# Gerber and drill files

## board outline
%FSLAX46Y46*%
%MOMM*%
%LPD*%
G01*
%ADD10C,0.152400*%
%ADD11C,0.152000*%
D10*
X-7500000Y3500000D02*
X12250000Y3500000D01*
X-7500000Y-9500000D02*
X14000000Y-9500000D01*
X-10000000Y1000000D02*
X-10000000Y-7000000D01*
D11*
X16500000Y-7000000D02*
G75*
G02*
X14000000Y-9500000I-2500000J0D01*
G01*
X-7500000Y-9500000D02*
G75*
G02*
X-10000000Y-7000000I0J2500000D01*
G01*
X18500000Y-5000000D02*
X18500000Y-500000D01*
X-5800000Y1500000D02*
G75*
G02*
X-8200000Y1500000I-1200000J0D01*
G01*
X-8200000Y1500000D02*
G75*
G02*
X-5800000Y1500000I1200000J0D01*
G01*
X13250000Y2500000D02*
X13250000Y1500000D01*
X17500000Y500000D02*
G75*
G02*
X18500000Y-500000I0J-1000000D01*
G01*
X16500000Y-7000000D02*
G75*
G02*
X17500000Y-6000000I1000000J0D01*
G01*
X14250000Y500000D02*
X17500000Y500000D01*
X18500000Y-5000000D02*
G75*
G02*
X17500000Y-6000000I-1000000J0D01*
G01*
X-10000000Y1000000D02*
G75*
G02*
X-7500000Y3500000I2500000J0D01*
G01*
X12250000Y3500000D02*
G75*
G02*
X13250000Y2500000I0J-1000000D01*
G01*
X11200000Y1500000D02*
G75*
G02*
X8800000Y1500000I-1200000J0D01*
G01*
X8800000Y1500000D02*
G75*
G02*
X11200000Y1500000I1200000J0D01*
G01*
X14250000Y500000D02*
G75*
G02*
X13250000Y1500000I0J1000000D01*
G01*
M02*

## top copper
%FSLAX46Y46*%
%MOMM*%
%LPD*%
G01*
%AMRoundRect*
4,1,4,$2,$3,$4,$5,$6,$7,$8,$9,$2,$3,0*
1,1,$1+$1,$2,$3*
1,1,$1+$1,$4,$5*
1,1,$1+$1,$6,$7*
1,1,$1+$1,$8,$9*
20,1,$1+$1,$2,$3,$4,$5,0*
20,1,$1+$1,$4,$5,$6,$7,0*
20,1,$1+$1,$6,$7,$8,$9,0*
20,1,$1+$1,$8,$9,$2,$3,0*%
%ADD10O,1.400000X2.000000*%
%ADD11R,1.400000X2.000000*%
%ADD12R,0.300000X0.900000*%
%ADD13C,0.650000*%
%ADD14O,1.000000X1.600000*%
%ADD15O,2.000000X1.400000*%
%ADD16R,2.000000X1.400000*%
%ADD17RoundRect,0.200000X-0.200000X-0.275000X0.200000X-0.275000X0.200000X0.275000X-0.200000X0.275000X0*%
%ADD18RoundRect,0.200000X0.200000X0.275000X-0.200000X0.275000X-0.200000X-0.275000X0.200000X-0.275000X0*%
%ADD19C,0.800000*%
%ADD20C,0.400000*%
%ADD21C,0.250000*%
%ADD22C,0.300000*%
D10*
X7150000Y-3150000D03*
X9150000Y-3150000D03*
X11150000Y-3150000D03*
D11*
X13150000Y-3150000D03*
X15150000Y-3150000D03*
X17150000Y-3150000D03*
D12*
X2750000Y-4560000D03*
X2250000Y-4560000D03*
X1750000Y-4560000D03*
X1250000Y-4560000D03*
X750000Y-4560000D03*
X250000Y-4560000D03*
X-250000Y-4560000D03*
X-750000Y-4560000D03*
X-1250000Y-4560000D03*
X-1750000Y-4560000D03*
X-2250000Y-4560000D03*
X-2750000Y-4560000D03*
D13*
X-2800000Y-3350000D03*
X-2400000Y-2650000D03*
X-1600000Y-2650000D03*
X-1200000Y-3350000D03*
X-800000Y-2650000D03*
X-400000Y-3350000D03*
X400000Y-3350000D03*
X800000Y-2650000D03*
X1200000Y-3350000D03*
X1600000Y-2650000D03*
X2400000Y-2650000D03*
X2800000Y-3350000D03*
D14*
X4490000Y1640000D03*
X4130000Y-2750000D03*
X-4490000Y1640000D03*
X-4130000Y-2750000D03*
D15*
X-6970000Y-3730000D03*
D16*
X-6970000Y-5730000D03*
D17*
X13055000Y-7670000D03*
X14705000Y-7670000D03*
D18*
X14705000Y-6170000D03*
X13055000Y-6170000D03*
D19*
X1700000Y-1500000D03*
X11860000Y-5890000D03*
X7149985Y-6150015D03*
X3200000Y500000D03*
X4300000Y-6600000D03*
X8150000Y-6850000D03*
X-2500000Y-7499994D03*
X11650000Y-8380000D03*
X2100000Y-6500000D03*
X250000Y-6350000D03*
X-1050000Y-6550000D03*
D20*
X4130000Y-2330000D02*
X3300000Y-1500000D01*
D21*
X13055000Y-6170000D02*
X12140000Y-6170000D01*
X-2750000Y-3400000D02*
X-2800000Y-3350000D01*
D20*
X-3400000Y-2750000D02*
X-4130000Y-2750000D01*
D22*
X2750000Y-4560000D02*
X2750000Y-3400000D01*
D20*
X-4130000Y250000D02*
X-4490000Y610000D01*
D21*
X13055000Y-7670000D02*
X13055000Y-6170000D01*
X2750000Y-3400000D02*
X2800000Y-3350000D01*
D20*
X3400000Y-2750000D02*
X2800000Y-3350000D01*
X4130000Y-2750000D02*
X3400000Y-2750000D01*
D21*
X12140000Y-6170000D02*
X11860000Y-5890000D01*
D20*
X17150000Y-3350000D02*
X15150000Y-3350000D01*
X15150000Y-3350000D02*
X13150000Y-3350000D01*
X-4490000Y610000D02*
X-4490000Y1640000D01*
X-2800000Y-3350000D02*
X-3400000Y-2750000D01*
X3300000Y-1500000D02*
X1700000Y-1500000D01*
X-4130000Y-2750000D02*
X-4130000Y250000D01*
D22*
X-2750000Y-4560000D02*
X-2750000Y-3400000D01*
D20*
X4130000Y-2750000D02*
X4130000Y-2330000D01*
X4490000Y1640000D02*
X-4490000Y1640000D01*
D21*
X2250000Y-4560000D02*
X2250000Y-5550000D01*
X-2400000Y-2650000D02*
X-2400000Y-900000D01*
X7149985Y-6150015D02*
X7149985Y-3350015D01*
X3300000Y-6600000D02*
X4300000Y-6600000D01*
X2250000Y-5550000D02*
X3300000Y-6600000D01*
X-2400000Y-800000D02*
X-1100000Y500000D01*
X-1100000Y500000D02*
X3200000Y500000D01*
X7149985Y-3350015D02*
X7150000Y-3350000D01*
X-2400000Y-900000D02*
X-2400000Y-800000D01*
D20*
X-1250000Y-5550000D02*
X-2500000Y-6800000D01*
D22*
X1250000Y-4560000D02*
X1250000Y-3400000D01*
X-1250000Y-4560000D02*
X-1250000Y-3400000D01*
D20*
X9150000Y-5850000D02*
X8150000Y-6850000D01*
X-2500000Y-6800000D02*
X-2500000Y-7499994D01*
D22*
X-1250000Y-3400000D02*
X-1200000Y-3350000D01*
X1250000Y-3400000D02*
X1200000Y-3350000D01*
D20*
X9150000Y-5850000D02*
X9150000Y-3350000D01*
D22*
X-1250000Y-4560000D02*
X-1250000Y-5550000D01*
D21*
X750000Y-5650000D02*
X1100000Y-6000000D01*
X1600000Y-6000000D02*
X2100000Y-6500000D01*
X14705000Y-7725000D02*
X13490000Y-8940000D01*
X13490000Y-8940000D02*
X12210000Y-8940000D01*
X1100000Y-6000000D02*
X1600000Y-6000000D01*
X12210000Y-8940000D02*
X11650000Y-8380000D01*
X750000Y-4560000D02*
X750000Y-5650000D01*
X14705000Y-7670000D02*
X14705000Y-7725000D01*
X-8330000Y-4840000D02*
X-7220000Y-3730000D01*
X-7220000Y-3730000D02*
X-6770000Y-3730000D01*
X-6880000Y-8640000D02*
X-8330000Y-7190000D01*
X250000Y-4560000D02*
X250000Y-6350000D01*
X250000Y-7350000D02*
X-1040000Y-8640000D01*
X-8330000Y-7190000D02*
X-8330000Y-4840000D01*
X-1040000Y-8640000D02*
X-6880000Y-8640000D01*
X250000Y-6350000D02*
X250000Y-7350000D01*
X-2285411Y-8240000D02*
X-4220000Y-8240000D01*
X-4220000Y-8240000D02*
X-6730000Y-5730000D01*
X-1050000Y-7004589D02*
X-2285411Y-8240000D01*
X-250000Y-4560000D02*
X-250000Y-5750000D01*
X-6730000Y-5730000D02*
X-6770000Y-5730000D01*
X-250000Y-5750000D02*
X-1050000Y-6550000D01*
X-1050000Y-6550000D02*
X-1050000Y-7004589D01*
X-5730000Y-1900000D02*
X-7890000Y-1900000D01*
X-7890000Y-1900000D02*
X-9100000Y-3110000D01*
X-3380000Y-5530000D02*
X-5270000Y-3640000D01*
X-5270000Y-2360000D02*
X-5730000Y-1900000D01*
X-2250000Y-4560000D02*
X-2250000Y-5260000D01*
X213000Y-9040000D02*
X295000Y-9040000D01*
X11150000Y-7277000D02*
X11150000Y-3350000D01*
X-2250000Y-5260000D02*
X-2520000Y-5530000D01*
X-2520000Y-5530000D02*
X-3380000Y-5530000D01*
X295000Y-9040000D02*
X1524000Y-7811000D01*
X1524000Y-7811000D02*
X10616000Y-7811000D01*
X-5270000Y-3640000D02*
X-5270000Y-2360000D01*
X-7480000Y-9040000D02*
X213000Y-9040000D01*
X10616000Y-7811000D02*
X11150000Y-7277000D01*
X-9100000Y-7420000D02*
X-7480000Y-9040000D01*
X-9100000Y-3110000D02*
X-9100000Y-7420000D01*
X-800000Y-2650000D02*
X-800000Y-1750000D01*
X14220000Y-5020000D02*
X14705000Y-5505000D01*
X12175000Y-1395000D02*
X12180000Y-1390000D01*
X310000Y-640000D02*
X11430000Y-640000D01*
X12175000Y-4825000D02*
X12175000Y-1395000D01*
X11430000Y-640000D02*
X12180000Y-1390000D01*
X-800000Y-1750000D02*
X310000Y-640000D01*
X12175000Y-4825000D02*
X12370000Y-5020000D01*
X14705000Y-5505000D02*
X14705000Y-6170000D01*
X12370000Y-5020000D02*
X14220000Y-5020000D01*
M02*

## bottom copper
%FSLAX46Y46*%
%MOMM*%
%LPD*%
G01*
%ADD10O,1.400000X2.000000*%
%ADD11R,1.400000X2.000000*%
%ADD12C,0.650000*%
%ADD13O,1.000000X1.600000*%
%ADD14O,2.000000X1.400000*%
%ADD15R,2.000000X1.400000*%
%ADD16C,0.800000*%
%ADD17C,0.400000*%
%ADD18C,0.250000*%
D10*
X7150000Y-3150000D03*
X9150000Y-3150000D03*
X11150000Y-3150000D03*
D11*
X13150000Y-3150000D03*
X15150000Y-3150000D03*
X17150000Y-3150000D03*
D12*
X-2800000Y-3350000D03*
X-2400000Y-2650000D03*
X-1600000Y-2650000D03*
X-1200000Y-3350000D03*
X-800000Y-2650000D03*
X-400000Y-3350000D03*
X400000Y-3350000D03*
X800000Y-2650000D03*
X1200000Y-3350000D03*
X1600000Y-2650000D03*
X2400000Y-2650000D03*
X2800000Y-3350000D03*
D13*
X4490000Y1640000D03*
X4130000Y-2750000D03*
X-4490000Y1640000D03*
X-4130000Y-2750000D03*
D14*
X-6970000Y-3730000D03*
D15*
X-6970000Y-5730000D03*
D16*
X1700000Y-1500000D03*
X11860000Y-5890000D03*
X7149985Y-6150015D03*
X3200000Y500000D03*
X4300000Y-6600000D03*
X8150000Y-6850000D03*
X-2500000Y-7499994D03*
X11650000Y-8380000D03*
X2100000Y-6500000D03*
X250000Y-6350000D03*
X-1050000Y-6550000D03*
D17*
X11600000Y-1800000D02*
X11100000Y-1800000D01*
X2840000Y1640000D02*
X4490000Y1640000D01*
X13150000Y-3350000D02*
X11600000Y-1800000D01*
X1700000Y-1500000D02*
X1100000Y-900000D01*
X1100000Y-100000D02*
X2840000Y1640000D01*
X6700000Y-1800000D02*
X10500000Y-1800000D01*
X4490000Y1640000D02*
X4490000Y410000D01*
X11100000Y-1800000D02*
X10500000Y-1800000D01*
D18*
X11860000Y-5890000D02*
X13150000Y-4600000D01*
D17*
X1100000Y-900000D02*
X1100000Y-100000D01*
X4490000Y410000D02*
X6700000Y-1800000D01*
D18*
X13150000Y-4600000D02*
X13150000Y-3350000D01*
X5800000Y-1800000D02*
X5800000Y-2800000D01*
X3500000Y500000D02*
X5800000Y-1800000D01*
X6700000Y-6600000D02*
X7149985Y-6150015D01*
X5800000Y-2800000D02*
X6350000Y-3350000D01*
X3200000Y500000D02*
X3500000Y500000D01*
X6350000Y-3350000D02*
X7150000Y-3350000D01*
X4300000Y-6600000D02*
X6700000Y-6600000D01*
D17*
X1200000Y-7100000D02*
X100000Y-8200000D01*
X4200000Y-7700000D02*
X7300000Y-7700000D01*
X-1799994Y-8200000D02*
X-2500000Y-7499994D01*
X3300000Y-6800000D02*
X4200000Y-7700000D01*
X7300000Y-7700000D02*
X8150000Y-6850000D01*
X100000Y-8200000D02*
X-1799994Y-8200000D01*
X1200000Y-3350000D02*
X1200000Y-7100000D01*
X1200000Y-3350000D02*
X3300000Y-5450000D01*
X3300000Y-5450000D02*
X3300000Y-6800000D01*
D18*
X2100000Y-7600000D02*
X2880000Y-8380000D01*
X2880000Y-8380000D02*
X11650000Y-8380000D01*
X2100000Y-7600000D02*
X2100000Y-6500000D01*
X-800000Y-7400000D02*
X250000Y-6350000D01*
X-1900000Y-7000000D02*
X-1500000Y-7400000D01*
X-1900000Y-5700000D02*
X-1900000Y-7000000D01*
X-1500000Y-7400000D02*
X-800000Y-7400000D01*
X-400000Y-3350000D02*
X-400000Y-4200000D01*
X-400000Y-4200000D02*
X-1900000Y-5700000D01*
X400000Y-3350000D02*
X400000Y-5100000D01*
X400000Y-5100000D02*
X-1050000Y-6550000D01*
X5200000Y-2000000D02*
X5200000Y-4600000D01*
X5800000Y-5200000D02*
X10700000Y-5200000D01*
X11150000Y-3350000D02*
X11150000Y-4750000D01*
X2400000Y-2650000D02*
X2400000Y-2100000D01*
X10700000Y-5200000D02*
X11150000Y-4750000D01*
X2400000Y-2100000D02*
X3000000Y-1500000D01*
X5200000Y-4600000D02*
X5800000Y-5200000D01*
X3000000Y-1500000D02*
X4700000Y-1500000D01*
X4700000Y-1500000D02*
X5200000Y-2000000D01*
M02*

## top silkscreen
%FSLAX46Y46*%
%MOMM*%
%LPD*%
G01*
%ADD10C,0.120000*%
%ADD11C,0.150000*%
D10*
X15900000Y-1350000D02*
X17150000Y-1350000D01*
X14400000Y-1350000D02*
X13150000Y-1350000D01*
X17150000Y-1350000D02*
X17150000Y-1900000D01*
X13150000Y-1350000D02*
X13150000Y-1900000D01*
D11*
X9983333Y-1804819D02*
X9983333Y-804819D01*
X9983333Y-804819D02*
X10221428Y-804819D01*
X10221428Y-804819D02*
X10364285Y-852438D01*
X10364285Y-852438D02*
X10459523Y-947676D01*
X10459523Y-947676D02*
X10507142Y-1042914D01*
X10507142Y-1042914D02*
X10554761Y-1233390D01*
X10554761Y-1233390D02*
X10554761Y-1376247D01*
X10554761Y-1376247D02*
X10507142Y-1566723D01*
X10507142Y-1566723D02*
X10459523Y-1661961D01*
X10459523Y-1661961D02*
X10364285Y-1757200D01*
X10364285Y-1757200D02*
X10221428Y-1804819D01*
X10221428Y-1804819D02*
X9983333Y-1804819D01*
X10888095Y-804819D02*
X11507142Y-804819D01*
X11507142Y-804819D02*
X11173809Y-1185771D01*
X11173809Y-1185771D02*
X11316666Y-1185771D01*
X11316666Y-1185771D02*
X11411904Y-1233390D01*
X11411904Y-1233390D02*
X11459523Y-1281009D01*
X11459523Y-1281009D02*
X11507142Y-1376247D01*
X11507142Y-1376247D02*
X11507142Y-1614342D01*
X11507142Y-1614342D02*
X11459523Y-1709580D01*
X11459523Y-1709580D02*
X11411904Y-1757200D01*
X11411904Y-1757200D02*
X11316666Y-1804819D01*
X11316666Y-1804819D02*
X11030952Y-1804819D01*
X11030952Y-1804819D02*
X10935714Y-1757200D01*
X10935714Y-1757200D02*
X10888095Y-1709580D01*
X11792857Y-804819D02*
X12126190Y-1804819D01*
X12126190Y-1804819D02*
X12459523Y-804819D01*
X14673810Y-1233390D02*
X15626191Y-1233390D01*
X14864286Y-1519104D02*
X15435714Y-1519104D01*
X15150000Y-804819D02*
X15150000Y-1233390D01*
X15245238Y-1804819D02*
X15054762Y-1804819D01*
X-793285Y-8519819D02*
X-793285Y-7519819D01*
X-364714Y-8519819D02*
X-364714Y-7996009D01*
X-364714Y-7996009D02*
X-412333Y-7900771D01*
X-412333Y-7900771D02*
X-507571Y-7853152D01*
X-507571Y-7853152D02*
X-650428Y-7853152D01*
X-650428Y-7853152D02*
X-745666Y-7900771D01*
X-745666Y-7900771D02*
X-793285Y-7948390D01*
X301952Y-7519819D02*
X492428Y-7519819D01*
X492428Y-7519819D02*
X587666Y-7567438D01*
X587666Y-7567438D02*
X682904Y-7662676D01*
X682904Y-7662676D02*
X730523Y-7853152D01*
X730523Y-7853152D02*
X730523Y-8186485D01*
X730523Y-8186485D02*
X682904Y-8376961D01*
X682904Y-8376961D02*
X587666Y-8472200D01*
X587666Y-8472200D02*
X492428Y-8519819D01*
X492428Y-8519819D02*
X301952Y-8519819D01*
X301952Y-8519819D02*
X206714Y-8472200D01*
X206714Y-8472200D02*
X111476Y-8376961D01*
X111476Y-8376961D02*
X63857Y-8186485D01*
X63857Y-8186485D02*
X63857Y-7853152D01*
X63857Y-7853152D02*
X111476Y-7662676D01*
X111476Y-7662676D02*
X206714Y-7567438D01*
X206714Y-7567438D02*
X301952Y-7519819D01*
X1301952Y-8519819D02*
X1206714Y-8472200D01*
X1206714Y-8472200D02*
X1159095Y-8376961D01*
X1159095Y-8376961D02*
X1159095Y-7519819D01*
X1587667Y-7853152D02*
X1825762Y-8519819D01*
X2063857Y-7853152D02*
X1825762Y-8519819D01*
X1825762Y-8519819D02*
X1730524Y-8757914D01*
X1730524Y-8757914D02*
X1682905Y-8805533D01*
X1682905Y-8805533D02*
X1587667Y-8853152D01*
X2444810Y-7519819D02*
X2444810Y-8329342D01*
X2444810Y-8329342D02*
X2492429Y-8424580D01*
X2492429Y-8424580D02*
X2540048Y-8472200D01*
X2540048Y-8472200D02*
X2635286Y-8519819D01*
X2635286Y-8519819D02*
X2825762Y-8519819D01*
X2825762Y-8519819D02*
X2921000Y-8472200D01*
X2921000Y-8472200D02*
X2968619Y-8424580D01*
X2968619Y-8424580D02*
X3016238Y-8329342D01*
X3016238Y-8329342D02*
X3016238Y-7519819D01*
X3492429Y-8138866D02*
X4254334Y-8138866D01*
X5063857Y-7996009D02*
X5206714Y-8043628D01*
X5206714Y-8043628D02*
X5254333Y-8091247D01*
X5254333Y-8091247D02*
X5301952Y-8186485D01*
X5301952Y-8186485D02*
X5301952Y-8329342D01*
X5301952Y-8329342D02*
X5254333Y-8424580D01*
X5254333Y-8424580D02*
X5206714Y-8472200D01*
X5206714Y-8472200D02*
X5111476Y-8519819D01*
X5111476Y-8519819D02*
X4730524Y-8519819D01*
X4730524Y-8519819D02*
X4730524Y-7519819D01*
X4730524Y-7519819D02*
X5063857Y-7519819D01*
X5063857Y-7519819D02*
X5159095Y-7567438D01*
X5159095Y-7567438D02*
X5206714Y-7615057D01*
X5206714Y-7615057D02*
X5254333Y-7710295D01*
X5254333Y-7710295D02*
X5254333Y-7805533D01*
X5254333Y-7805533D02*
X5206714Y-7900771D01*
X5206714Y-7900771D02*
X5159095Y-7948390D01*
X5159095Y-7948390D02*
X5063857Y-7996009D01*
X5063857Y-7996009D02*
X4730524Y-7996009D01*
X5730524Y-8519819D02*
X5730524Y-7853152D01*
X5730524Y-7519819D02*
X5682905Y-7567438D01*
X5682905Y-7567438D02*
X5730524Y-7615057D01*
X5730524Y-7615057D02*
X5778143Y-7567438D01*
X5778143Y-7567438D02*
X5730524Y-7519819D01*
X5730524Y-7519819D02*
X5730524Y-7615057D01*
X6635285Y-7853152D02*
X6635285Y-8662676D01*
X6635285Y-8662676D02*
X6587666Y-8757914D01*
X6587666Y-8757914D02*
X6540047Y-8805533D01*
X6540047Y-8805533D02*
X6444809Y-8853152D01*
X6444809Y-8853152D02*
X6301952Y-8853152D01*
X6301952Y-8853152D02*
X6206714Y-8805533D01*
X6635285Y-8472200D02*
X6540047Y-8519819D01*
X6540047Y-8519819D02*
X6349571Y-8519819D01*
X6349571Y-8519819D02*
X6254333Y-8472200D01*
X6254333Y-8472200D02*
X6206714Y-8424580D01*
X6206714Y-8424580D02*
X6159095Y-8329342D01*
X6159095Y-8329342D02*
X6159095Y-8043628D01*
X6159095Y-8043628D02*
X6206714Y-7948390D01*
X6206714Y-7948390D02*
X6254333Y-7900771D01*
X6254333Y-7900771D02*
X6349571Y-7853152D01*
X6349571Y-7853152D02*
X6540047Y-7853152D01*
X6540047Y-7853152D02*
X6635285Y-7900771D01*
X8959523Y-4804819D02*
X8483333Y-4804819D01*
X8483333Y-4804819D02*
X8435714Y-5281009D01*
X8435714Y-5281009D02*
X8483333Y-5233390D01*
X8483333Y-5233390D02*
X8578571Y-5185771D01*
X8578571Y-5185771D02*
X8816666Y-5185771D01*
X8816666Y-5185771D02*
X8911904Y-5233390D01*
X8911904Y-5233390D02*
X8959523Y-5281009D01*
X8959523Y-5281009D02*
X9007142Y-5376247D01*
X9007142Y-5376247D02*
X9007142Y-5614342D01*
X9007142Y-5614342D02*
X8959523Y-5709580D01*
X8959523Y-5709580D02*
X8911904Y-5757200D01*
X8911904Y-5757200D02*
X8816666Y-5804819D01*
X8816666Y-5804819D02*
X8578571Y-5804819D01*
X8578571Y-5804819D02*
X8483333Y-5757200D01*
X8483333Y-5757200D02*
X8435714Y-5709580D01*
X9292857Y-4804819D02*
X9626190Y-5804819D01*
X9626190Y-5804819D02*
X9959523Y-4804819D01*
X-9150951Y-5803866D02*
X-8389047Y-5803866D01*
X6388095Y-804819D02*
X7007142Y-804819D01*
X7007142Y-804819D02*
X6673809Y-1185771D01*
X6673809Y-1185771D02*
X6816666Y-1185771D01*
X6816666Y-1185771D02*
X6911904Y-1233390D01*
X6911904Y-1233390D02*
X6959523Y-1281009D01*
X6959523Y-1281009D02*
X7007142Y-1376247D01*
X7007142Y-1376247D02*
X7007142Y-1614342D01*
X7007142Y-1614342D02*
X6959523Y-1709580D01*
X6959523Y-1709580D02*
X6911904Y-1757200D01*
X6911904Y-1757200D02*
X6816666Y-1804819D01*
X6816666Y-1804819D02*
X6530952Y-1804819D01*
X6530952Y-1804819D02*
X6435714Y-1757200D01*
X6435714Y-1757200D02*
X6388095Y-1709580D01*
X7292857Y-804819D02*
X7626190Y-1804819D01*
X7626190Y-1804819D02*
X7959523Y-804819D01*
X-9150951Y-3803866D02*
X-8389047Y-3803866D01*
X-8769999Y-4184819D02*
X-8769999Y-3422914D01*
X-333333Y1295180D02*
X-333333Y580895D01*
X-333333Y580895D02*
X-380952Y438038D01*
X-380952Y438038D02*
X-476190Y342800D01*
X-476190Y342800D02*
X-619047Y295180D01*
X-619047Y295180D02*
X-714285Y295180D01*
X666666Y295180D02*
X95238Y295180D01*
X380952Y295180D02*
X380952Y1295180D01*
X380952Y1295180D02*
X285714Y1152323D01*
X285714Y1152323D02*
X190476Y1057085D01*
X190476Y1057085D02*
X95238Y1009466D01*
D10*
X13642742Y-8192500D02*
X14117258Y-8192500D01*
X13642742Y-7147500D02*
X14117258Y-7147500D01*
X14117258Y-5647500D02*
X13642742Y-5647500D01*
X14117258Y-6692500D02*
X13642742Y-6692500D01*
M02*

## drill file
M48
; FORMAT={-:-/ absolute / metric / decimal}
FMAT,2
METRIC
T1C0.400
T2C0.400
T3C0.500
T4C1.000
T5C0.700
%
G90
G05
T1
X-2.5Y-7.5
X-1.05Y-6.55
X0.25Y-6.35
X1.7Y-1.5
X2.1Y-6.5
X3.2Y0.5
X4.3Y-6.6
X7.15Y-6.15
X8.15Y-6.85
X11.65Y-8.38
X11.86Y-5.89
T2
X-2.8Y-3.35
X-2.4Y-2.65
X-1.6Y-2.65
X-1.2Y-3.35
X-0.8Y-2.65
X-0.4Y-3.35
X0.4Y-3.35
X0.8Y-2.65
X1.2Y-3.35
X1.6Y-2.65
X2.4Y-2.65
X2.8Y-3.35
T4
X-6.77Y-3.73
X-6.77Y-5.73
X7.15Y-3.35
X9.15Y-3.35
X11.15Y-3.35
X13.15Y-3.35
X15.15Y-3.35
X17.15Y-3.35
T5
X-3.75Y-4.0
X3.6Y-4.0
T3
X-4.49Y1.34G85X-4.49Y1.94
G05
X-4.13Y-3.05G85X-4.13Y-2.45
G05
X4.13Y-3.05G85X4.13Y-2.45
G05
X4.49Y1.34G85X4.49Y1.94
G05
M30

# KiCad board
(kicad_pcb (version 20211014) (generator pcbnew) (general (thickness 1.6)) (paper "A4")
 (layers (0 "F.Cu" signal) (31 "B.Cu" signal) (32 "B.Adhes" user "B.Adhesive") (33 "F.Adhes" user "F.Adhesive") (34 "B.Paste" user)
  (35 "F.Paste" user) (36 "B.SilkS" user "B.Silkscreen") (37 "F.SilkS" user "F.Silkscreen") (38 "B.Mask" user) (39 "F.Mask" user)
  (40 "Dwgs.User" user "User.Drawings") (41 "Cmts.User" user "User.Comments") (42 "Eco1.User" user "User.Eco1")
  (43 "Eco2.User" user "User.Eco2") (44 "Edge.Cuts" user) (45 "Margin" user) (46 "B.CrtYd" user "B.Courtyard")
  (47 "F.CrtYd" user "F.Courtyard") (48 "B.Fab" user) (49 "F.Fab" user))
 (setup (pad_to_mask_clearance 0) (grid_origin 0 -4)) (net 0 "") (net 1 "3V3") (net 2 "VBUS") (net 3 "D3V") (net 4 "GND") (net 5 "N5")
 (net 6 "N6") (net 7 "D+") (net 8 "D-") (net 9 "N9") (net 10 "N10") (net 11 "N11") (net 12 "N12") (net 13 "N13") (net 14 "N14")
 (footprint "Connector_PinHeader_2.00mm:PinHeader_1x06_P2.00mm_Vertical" (layer "F.Cu") (at 7.15 3.35 90)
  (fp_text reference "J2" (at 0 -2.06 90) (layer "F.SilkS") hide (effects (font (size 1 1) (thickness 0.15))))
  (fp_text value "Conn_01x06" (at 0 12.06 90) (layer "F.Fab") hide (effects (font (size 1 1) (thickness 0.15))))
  (pad "1" thru_hole oval locked (at 0 0 90) (size 2 1.4) (drill 1 (offset 0.2 0)) (layers *.Cu *.Mask) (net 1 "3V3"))
  (pad "2" thru_hole oval locked (at 0 2 90) (size 2 1.4) (drill 1 (offset 0.2 0)) (layers *.Cu *.Mask) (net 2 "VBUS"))
  (pad "3" thru_hole oval locked (at 0 4 90) (size 2 1.4) (drill 1 (offset 0.2 0)) (layers *.Cu *.Mask) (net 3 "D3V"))
  (pad "4" thru_hole rect locked (at 0 6 90) (size 2 1.4) (drill 1 (offset 0.2 0)) (layers *.Cu *.Mask) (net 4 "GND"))
  (pad "5" thru_hole rect locked (at 0 8 90) (size 2 1.4) (drill 1 (offset 0.2 0)) (layers *.Cu *.Mask) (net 4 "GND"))
  (pad "6" thru_hole rect locked (at 0 10 90) (size 2 1.4) (drill 1 (offset 0.2 0)) (layers *.Cu *.Mask) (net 4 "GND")))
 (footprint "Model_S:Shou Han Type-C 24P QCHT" (layer "F.Cu") (at 0 -3.5 180)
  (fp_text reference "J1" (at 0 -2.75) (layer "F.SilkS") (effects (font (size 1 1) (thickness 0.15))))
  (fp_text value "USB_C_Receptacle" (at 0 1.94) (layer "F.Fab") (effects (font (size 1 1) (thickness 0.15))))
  (pad "" np_thru_hole circle locked (at -3.6 -7.5 180) (size 0.7 0.7) (drill 0.7) (layers *.Cu *.Mask))
  (pad "" np_thru_hole circle locked (at 3.75 -7.5 180) (size 0.7 0.7) (drill 0.7) (layers *.Cu *.Mask))
  (pad "A1" smd rect locked (at -2.75 -8.06 180) (size 0.3 0.9) (layers "F.Cu" "F.Paste" "F.Mask") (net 4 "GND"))
  (pad "A2" smd rect locked (at -2.25 -8.06 180) (size 0.3 0.9) (layers "F.Cu" "F.Paste" "F.Mask") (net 1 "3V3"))
  (pad "A3" smd rect locked (at -1.75 -8.06 180) (size 0.3 0.9) (layers "F.Cu" "F.Paste" "F.Mask") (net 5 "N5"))
  (pad "A4" smd rect locked (at -1.25 -8.06 180) (size 0.3 0.9) (layers "F.Cu" "F.Paste" "F.Mask") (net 2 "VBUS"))
  (pad "A5" smd rect locked (at -0.75 -8.06 180) (size 0.3 0.9) (layers "F.Cu" "F.Paste" "F.Mask") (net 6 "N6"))
  (pad "A6" smd rect locked (at -0.25 -8.06 180) (size 0.3 0.9) (layers "F.Cu" "F.Paste" "F.Mask") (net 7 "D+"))
  (pad "A7" smd rect locked (at 0.25 -8.06 180) (size 0.3 0.9) (layers "F.Cu" "F.Paste" "F.Mask") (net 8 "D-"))
  (pad "A8" smd rect locked (at 0.75 -8.06 180) (size 0.3 0.9) (layers "F.Cu" "F.Paste" "F.Mask") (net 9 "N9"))
  (pad "A9" smd rect locked (at 1.25 -8.06 180) (size 0.3 0.9) (layers "F.Cu" "F.Paste" "F.Mask") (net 2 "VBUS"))
  (pad "A10" smd rect locked (at 1.75 -8.06 180) (size 0.3 0.9) (layers "F.Cu" "F.Paste" "F.Mask") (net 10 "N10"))
  (pad "A11" smd rect locked (at 2.25 -8.06 180) (size 0.3 0.9) (layers "F.Cu" "F.Paste" "F.Mask") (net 3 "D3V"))
  (pad "A12" smd rect locked (at 2.75 -8.06 180) (size 0.3 0.9) (layers "F.Cu" "F.Paste" "F.Mask") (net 4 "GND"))
  (pad "B1" thru_hole circle locked (at 2.8 -6.85 180) (size 0.65 0.65) (drill 0.4) (layers *.Cu *.Mask) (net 4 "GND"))
  (pad "B2" thru_hole circle locked (at 2.4 -6.15 180) (size 0.65 0.65) (drill 0.4) (layers *.Cu *.Mask) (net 1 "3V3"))
  (pad "B3" thru_hole circle locked (at 1.6 -6.15 180) (size 0.65 0.65) (drill 0.4) (layers *.Cu *.Mask) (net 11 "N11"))
  (pad "B4" thru_hole circle locked (at 1.2 -6.85 180) (size 0.65 0.65) (drill 0.4) (layers *.Cu *.Mask) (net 2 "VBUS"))
  (pad "B5" thru_hole circle locked (at 0.8 -6.15 180) (size 0.65 0.65) (drill 0.4) (layers *.Cu *.Mask) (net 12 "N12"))
  (pad "B6" thru_hole circle locked (at 0.4 -6.85 180) (size 0.65 0.65) (drill 0.4) (layers *.Cu *.Mask) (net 7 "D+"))
  (pad "B7" thru_hole circle locked (at -0.4 -6.85 180) (size 0.65 0.65) (drill 0.4) (layers *.Cu *.Mask) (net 8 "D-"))
  (pad "B8" thru_hole circle locked (at -0.8 -6.15 180) (size 0.65 0.65) (drill 0.4) (layers *.Cu *.Mask) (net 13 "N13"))
  (pad "B9" thru_hole circle locked (at -1.2 -6.85 180) (size 0.65 0.65) (drill 0.4) (layers *.Cu *.Mask) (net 2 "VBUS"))
  (pad "B10" thru_hole circle locked (at -1.6 -6.15 180) (size 0.65 0.65) (drill 0.4) (layers *.Cu *.Mask) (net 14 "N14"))
  (pad "B11" thru_hole circle locked (at -2.4 -6.15 180) (size 0.65 0.65) (drill 0.4) (layers *.Cu *.Mask) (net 3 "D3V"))
  (pad "B12" thru_hole circle locked (at -2.8 -6.85 180) (size 0.65 0.65) (drill 0.4) (layers *.Cu *.Mask) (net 4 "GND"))
  (pad "S1" thru_hole oval locked (at -4.49 -1.86 180) (size 1 1.6) (drill oval 0.5 1.1) (layers *.Cu *.Mask) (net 4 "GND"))
  (pad "S1" thru_hole oval locked (at -4.13 -6.25 180) (size 1 1.6) (drill oval 0.5 1.1) (layers *.Cu *.Mask) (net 4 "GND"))
  (pad "S1" thru_hole oval locked (at 4.49 -1.86 180) (size 1 1.6) (drill oval 0.5 1.1) (layers *.Cu *.Mask) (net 4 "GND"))
  (pad "S1" thru_hole oval locked (at 4.13 -6.25 180) (size 1 1.6) (drill oval 0.5 1.1) (layers *.Cu *.Mask) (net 4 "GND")))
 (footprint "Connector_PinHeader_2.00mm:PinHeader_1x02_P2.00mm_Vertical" (layer "F.Cu") (at -6.77 3.73)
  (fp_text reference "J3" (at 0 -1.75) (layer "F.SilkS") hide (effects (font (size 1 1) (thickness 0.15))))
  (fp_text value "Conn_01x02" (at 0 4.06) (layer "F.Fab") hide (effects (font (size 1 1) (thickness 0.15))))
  (pad "1" thru_hole oval locked (at 0 0) (size 2 1.4) (drill 1 (offset -0.2 0)) (layers *.Cu *.Mask) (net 7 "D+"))
  (pad "2" thru_hole rect locked (at 0 2) (size 2 1.4) (drill 1 (offset -0.2 0)) (layers *.Cu *.Mask) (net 8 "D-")))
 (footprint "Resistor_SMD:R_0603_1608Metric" (layer "F.Cu") (at 13.88 7.67)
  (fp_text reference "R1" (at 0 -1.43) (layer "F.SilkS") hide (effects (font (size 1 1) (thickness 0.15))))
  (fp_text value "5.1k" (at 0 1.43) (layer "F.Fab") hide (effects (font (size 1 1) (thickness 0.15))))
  (fp_line (start -0.237258 0.5225) (end 0.237258 0.5225) (layer "F.SilkS") (width 0.12))
  (fp_line (start -0.237258 -0.5225) (end 0.237258 -0.5225) (layer "F.SilkS") (width 0.12))
  (pad "1" smd roundrect locked (at -0.825 0) (size 0.8 0.95) (layers "F.Cu" "F.Paste" "F.Mask") (roundrect_rratio 0.25) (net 4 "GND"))
  (pad "2" smd roundrect locked (at 0.825 0) (size 0.8 0.95) (layers "F.Cu" "F.Paste" "F.Mask") (roundrect_rratio 0.25) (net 6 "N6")))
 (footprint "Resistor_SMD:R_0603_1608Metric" (layer "F.Cu") (at 13.88 6.17 180)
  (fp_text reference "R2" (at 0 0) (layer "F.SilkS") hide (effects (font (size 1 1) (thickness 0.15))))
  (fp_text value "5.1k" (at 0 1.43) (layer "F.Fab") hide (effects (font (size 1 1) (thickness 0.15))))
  (fp_line (start -0.237258 0.5225) (end 0.237258 0.5225) (layer "F.SilkS") (width 0.12))
  (fp_line (start -0.237258 -0.5225) (end 0.237258 -0.5225) (layer "F.SilkS") (width 0.12))
  (pad "1" smd roundrect locked (at -0.825 0 180) (size 0.8 0.95) (layers "F.Cu" "F.Paste" "F.Mask") (roundrect_rratio 0.25) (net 12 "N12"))
  (pad "2" smd roundrect locked (at 0.825 0 180) (size 0.8 0.95) (layers "F.Cu" "F.Paste" "F.Mask") (roundrect_rratio 0.25) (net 4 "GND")))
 (gr_line (start 15.9 1.35) (end 17.15 1.35) (layer "F.SilkS") (width 0.12))
 (gr_line (start 14.4 1.35) (end 13.15 1.35) (layer "F.SilkS") (width 0.12))
 (gr_line (start 17.15 1.35) (end 17.15 1.9) (layer "F.SilkS") (width 0.12))
 (gr_line (start 13.15 1.35) (end 13.15 1.9) (layer "F.SilkS") (width 0.12))
 (gr_line (start -7.5 -3.5) (end 12.25 -3.5) (layer "Edge.Cuts") (width 0.1524))
 (gr_line (start -7.5 9.5) (end 14 9.5) (layer "Edge.Cuts") (width 0.1524))
 (gr_line (start -10 -1) (end -10 7) (layer "Edge.Cuts") (width 0.1524))
 (gr_arc (start 16.5 7) (mid 15.767767 8.767767) (end 14 9.5) (layer "Edge.Cuts") (width 0.152))
 (gr_arc (start -7.5 9.5) (mid -9.267767 8.767767) (end -10 7) (layer "Edge.Cuts") (width 0.152))
 (gr_line (start 18.5 5) (end 18.5 0.5) (layer "Edge.Cuts") (width 0.152))
 (gr_circle (center -7 -1.5) (end -5.8 -1.5) (layer "Edge.Cuts") (width 0.152) (fill none))
 (gr_line (start 13.25 -2.5) (end 13.25 -1.5) (layer "Edge.Cuts") (width 0.152))
 (gr_arc (start 17.5 -0.5) (mid 18.207107 -0.207107) (end 18.5 0.5) (layer "Edge.Cuts") (width 0.152))
 (gr_arc (start 16.5 7) (mid 16.792893 6.292893) (end 17.5 6) (layer "Edge.Cuts") (width 0.152))
 (gr_line (start 14.25 -0.5) (end 17.5 -0.5) (layer "Edge.Cuts") (width 0.152))
 (gr_arc (start 18.5 5) (mid 18.207107 5.707107) (end 17.5 6) (layer "Edge.Cuts") (width 0.152))
 (gr_arc (start -10 -1) (mid -9.267767 -2.767767) (end -7.5 -3.5) (layer "Edge.Cuts") (width 0.152))
 (gr_arc (start 12.25 -3.5) (mid 12.957107 -3.207107) (end 13.25 -2.5) (layer "Edge.Cuts") (width 0.152))
 (gr_circle (center 10 -1.5) (end 11.2 -1.5) (layer "Edge.Cuts") (width 0.152) (fill none))
 (gr_arc (start 14.25 -0.5) (mid 13.542893 -0.792893) (end 13.25 -1.5) (layer "Edge.Cuts") (width 0.152))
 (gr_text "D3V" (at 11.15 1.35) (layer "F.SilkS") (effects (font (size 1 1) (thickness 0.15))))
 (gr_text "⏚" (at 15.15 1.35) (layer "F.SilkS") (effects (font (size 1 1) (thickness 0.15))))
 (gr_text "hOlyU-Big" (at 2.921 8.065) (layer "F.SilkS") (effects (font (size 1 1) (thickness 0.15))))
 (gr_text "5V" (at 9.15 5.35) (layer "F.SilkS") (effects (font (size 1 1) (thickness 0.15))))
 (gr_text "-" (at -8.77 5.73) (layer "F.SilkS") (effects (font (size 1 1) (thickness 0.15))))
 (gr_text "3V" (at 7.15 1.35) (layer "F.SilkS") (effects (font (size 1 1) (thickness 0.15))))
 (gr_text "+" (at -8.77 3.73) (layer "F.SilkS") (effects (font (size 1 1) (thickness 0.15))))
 (segment (start 4.13 2.33) (end 3.3 1.5) (width 0.4) (layer "F.Cu") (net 4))
 (segment (start 13.055 6.17) (end 12.14 6.17) (width 0.25) (layer "F.Cu") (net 4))
 (segment (start -2.75 3.4) (end -2.8 3.35) (width 0.25) (layer "F.Cu") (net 4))
 (segment (start -3.4 2.75) (end -4.13 2.75) (width 0.4) (layer "F.Cu") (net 4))
 (segment (start 2.75 4.56) (end 2.75 3.4) (width 0.3) (layer "F.Cu") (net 4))
 (segment (start -4.13 -0.25) (end -4.49 -0.61) (width 0.4) (layer "F.Cu") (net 4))
 (segment (start 13.055 7.67) (end 13.055 6.17) (width 0.25) (layer "F.Cu") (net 4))
 (segment (start 2.75 3.4) (end 2.8 3.35) (width 0.25) (layer "F.Cu") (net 4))
 (segment (start 3.4 2.75) (end 2.8 3.35) (width 0.4) (layer "F.Cu") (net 4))
 (segment (start 4.13 2.75) (end 3.4 2.75) (width 0.4) (layer "F.Cu") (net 4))
 (segment (start 12.14 6.17) (end 11.86 5.89) (width 0.25) (layer "F.Cu") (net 4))
 (segment (start 17.15 3.35) (end 15.15 3.35) (width 0.4) (layer "F.Cu") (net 4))
 (segment (start 15.15 3.35) (end 13.15 3.35) (width 0.4) (layer "F.Cu") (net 4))
 (segment (start -4.49 -0.61) (end -4.49 -1.64) (width 0.4) (layer "F.Cu") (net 4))
 (segment (start -2.8 3.35) (end -3.4 2.75) (width 0.4) (layer "F.Cu") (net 4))
 (segment (start 3.3 1.5) (end 1.7 1.5) (width 0.4) (layer "F.Cu") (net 4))
 (segment (start -4.13 2.75) (end -4.13 -0.25) (width 0.4) (layer "F.Cu") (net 4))
 (segment (start -2.75 4.56) (end -2.75 3.4) (width 0.3) (layer "F.Cu") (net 4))
 (segment (start 4.13 2.75) (end 4.13 2.33) (width 0.4) (layer "F.Cu") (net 4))
 (segment (start 4.49 -1.64) (end -4.49 -1.64) (width 0.4) (layer "F.Cu") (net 4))
 (via (at 1.7 1.5) (size 0.8) (drill 0.4) (layers "F.Cu" "B.Cu") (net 4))
 (via (at 11.86 5.89) (size 0.8) (drill 0.4) (layers "F.Cu" "B.Cu") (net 4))
 (segment (start 11.6 1.8) (end 11.1 1.8) (width 0.4) (layer "B.Cu") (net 4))
 (segment (start 2.84 -1.64) (end 4.49 -1.64) (width 0.4) (layer "B.Cu") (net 4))
 (segment (start 13.15 3.35) (end 11.6 1.8) (width 0.4) (layer "B.Cu") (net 4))
 (segment (start 1.7 1.5) (end 1.1 0.9) (width 0.4) (layer "B.Cu") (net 4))
 (segment (start 1.1 0.1) (end 2.84 -1.64) (width 0.4) (layer "B.Cu") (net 4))
 (segment (start 6.7 1.8) (end 10.5 1.8) (width 0.4) (layer "B.Cu") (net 4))
 (segment (start 4.49 -1.64) (end 4.49 -0.41) (width 0.4) (layer "B.Cu") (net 4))
 (segment (start 11.1 1.8) (end 10.5 1.8) (width 0.4) (layer "B.Cu") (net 4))
 (segment (start 11.86 5.89) (end 13.15 4.6) (width 0.25) (layer "B.Cu") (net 4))
 (segment (start 1.1 0.9) (end 1.1 0.1) (width 0.4) (layer "B.Cu") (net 4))
 (segment (start 4.49 -0.41) (end 6.7 1.8) (width 0.4) (layer "B.Cu") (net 4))
 (segment (start 13.15 4.6) (end 13.15 3.35) (width 0.25) (layer "B.Cu") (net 4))
 (segment (start 2.25 4.56) (end 2.25 5.55) (width 0.25) (layer "F.Cu") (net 1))
 (segment (start -2.4 2.65) (end -2.4 0.9) (width 0.25) (layer "F.Cu") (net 1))
 (segment (start 7.149985 6.150015) (end 7.149985 3.350015) (width 0.25) (layer "F.Cu") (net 1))
 (segment (start 3.3 6.6) (end 4.3 6.6) (width 0.25) (layer "F.Cu") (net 1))
 (segment (start 2.25 5.55) (end 3.3 6.6) (width 0.25) (layer "F.Cu") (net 1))
 (segment (start -2.4 0.8) (end -1.1 -0.5) (width 0.25) (layer "F.Cu") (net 1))
 (segment (start -1.1 -0.5) (end 3.2 -0.5) (width 0.25) (layer "F.Cu") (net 1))
 (segment (start 7.149985 3.350015) (end 7.15 3.35) (width 0.25) (layer "F.Cu") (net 1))
 (segment (start -2.4 0.9) (end -2.4 0.8) (width 0.25) (layer "F.Cu") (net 1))
 (via (at 7.149985 6.150015) (size 0.8) (drill 0.4) (layers "F.Cu" "B.Cu") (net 1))
 (via (at 3.2 -0.5) (size 0.8) (drill 0.4) (layers "F.Cu" "B.Cu") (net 1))
 (via (at 4.3 6.6) (size 0.8) (drill 0.4) (layers "F.Cu" "B.Cu") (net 1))
 (segment (start 5.8 1.8) (end 5.8 2.8) (width 0.25) (layer "B.Cu") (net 1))
 (segment (start 3.5 -0.5) (end 5.8 1.8) (width 0.25) (layer "B.Cu") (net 1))
 (segment (start 6.7 6.6) (end 7.149985 6.150015) (width 0.25) (layer "B.Cu") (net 1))
 (segment (start 5.8 2.8) (end 6.35 3.35) (width 0.25) (layer "B.Cu") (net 1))
 (segment (start 3.2 -0.5) (end 3.5 -0.5) (width 0.25) (layer "B.Cu") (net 1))
 (segment (start 6.35 3.35) (end 7.15 3.35) (width 0.25) (layer "B.Cu") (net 1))
 (segment (start 4.3 6.6) (end 6.7 6.6) (width 0.25) (layer "B.Cu") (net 1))
 (segment (start -1.25 5.55) (end -2.5 6.8) (width 0.4) (layer "F.Cu") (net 2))
 (segment (start 1.25 4.56) (end 1.25 3.4) (width 0.3) (layer "F.Cu") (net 2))
 (segment (start -1.25 4.56) (end -1.25 3.4) (width 0.3) (layer "F.Cu") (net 2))
 (segment (start 9.15 5.85) (end 8.15 6.85) (width 0.4) (layer "F.Cu") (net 2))
 (segment (start -2.5 6.8) (end -2.5 7.499994) (width 0.4) (layer "F.Cu") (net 2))
 (segment (start -1.25 3.4) (end -1.2 3.35) (width 0.3) (layer "F.Cu") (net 2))
 (segment (start 1.25 3.4) (end 1.2 3.35) (width 0.3) (layer "F.Cu") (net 2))
 (segment (start 9.15 5.85) (end 9.15 3.35) (width 0.4) (layer "F.Cu") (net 2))
 (segment (start -1.25 4.56) (end -1.25 5.55) (width 0.3) (layer "F.Cu") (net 2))
 (via (at 8.15 6.85) (size 0.8) (drill 0.4) (layers "F.Cu" "B.Cu") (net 2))
 (via (at -2.5 7.499994) (size 0.8) (drill 0.4) (layers "F.Cu" "B.Cu") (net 2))
 (segment (start 1.2 7.1) (end 0.1 8.2) (width 0.4) (layer "B.Cu") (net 2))
 (segment (start 4.2 7.7) (end 7.3 7.7) (width 0.4) (layer "B.Cu") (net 2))
 (segment (start -1.799994 8.2) (end -2.5 7.499994) (width 0.4) (layer "B.Cu") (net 2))
 (segment (start 3.3 6.8) (end 4.2 7.7) (width 0.4) (layer "B.Cu") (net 2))
 (segment (start 7.3 7.7) (end 8.15 6.85) (width 0.4) (layer "B.Cu") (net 2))
 (segment (start 0.1 8.2) (end -1.799994 8.2) (width 0.4) (layer "B.Cu") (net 2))
 (segment (start 1.2 3.35) (end 1.2 7.1) (width 0.4) (layer "B.Cu") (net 2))
 (segment (start 1.2 3.35) (end 3.3 5.45) (width 0.4) (layer "B.Cu") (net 2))
 (segment (start 3.3 5.45) (end 3.3 6.8) (width 0.4) (layer "B.Cu") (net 2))
 (segment (start 0.75 5.65) (end 1.1 6) (width 0.25) (layer "F.Cu") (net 6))
 (segment (start 1.6 6) (end 2.1 6.5) (width 0.25) (layer "F.Cu") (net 6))
 (segment (start 14.705 7.725) (end 13.49 8.94) (width 0.25) (layer "F.Cu") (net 6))
 (segment (start 13.49 8.94) (end 12.21 8.94) (width 0.25) (layer "F.Cu") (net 6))
 (segment (start 1.1 6) (end 1.6 6) (width 0.25) (layer "F.Cu") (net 6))
 (segment (start 12.21 8.94) (end 11.65 8.38) (width 0.25) (layer "F.Cu") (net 6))
 (segment (start 0.75 4.56) (end 0.75 5.65) (width 0.25) (layer "F.Cu") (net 6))
 (segment (start 14.705 7.67) (end 14.705 7.725) (width 0.25) (layer "F.Cu") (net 6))
 (via (at 11.65 8.38) (size 0.8) (drill 0.4) (layers "F.Cu" "B.Cu") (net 6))
 (via (at 2.1 6.5) (size 0.8) (drill 0.4) (layers "F.Cu" "B.Cu") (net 6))
 (segment (start 2.1 7.6) (end 2.88 8.38) (width 0.25) (layer "B.Cu") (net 6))
 (segment (start 2.88 8.38) (end 11.65 8.38) (width 0.25) (layer "B.Cu") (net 6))
 (segment (start 2.1 7.6) (end 2.1 6.5) (width 0.25) (layer "B.Cu") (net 6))
 (segment (start -8.33 4.84) (end -7.22 3.73) (width 0.25) (layer "F.Cu") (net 7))
 (segment (start -7.22 3.73) (end -6.77 3.73) (width 0.25) (layer "F.Cu") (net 7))
 (segment (start -6.88 8.64) (end -8.33 7.19) (width 0.25) (layer "F.Cu") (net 7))
 (segment (start 0.25 4.56) (end 0.25 6.35) (width 0.25) (layer "F.Cu") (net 7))
 (segment (start 0.25 7.35) (end -1.04 8.64) (width 0.25) (layer "F.Cu") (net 7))
 (segment (start -8.33 7.19) (end -8.33 4.84) (width 0.25) (layer "F.Cu") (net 7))
 (segment (start -1.04 8.64) (end -6.88 8.64) (width 0.25) (layer "F.Cu") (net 7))
 (segment (start 0.25 6.35) (end 0.25 7.35) (width 0.25) (layer "F.Cu") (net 7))
 (via (at 0.25 6.35) (size 0.8) (drill 0.4) (layers "F.Cu" "B.Cu") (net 7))
 (segment (start -0.8 7.4) (end 0.25 6.35) (width 0.25) (layer "B.Cu") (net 7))
 (segment (start -1.9 7) (end -1.5 7.4) (width 0.25) (layer "B.Cu") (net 7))
 (segment (start -1.9 5.7) (end -1.9 7) (width 0.25) (layer "B.Cu") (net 7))
 (segment (start -1.5 7.4) (end -0.8 7.4) (width 0.25) (layer "B.Cu") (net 7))
 (segment (start -0.4 3.35) (end -0.4 4.2) (width 0.25) (layer "B.Cu") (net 7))
 (segment (start -0.4 4.2) (end -1.9 5.7) (width 0.25) (layer "B.Cu") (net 7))
 (segment (start -2.285411 8.24) (end -4.22 8.24) (width 0.25) (layer "F.Cu") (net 8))
 (segment (start -4.22 8.24) (end -6.73 5.73) (width 0.25) (layer "F.Cu") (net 8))
 (segment (start -1.05 7.004589) (end -2.285411 8.24) (width 0.25) (layer "F.Cu") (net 8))
 (segment (start -0.25 4.56) (end -0.25 5.75) (width 0.25) (layer "F.Cu") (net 8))
 (segment (start -6.73 5.73) (end -6.77 5.73) (width 0.25) (layer "F.Cu") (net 8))
 (segment (start -0.25 5.75) (end -1.05 6.55) (width 0.25) (layer "F.Cu") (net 8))
 (segment (start -1.05 6.55) (end -1.05 7.004589) (width 0.25) (layer "F.Cu") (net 8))
 (via (at -1.05 6.55) (size 0.8) (drill 0.4) (layers "F.Cu" "B.Cu") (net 8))
 (segment (start 0.4 3.35) (end 0.4 5.1) (width 0.25) (layer "B.Cu") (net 8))
 (segment (start 0.4 5.1) (end -1.05 6.55) (width 0.25) (layer "B.Cu") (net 8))
 (segment (start -5.73 1.9) (end -7.89 1.9) (width 0.25) (layer "F.Cu") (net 3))
 (segment (start -7.89 1.9) (end -9.1 3.11) (width 0.25) (layer "F.Cu") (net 3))
 (segment (start -3.38 5.53) (end -5.27 3.64) (width 0.25) (layer "F.Cu") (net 3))
 (segment (start -5.27 2.36) (end -5.73 1.9) (width 0.25) (layer "F.Cu") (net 3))
 (segment (start -2.25 4.56) (end -2.25 5.26) (width 0.25) (layer "F.Cu") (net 3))
 (segment (start 0.213 9.04) (end 0.295 9.04) (width 0.25) (layer "F.Cu") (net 3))
 (segment (start 11.15 7.277) (end 11.15 3.35) (width 0.25) (layer "F.Cu") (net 3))
 (segment (start -2.25 5.26) (end -2.52 5.53) (width 0.25) (layer "F.Cu") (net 3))
 (segment (start -2.52 5.53) (end -3.38 5.53) (width 0.25) (layer "F.Cu") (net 3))
 (segment (start 0.295 9.04) (end 1.524 7.811) (width 0.25) (layer "F.Cu") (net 3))
 (segment (start 1.524 7.811) (end 10.616 7.811) (width 0.25) (layer "F.Cu") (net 3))
 (segment (start -5.27 3.64) (end -5.27 2.36) (width 0.25) (layer "F.Cu") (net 3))
 (segment (start -7.48 9.04) (end 0.213 9.04) (width 0.25) (layer "F.Cu") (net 3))
 (segment (start 10.616 7.811) (end 11.15 7.277) (width 0.25) (layer "F.Cu") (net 3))
 (segment (start -9.1 7.42) (end -7.48 9.04) (width 0.25) (layer "F.Cu") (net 3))
 (segment (start -9.1 3.11) (end -9.1 7.42) (width 0.25) (layer "F.Cu") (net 3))
 (segment (start 5.2 2) (end 5.2 4.6) (width 0.25) (layer "B.Cu") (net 3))
 (segment (start 5.8 5.2) (end 10.7 5.2) (width 0.25) (layer "B.Cu") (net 3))
 (segment (start 11.15 3.35) (end 11.15 4.75) (width 0.25) (layer "B.Cu") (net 3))
 (segment (start 2.4 2.65) (end 2.4 2.1) (width 0.25) (layer "B.Cu") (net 3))
 (segment (start 10.7 5.2) (end 11.15 4.75) (width 0.25) (layer "B.Cu") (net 3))
 (segment (start 2.4 2.1) (end 3 1.5) (width 0.25) (layer "B.Cu") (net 3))
 (segment (start 5.2 4.6) (end 5.8 5.2) (width 0.25) (layer "B.Cu") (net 3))
 (segment (start 3 1.5) (end 4.7 1.5) (width 0.25) (layer "B.Cu") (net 3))
 (segment (start 4.7 1.5) (end 5.2 2) (width 0.25) (layer "B.Cu") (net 3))
 (segment (start -0.8 2.65) (end -0.8 1.75) (width 0.25) (layer "F.Cu") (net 12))
 (segment (start 14.22 5.02) (end 14.705 5.505) (width 0.25) (layer "F.Cu") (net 12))
 (segment (start 12.175 1.395) (end 12.18 1.39) (width 0.25) (layer "F.Cu") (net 12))
 (segment (start 0.31 0.64) (end 11.43 0.64) (width 0.25) (layer "F.Cu") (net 12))
 (segment (start 12.175 4.825) (end 12.175 1.395) (width 0.25) (layer "F.Cu") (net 12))
 (segment (start 11.43 0.64) (end 12.18 1.39) (width 0.25) (layer "F.Cu") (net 12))
 (segment (start -0.8 1.75) (end 0.31 0.64) (width 0.25) (layer "F.Cu") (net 12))
 (segment (start 12.175 4.825) (end 12.37 5.02) (width 0.25) (layer "F.Cu") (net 12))
 (segment (start 14.705 5.505) (end 14.705 6.17) (width 0.25) (layer "F.Cu") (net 12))
 (segment (start 12.37 5.02) (end 14.22 5.02) (width 0.25) (layer "F.Cu") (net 12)))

